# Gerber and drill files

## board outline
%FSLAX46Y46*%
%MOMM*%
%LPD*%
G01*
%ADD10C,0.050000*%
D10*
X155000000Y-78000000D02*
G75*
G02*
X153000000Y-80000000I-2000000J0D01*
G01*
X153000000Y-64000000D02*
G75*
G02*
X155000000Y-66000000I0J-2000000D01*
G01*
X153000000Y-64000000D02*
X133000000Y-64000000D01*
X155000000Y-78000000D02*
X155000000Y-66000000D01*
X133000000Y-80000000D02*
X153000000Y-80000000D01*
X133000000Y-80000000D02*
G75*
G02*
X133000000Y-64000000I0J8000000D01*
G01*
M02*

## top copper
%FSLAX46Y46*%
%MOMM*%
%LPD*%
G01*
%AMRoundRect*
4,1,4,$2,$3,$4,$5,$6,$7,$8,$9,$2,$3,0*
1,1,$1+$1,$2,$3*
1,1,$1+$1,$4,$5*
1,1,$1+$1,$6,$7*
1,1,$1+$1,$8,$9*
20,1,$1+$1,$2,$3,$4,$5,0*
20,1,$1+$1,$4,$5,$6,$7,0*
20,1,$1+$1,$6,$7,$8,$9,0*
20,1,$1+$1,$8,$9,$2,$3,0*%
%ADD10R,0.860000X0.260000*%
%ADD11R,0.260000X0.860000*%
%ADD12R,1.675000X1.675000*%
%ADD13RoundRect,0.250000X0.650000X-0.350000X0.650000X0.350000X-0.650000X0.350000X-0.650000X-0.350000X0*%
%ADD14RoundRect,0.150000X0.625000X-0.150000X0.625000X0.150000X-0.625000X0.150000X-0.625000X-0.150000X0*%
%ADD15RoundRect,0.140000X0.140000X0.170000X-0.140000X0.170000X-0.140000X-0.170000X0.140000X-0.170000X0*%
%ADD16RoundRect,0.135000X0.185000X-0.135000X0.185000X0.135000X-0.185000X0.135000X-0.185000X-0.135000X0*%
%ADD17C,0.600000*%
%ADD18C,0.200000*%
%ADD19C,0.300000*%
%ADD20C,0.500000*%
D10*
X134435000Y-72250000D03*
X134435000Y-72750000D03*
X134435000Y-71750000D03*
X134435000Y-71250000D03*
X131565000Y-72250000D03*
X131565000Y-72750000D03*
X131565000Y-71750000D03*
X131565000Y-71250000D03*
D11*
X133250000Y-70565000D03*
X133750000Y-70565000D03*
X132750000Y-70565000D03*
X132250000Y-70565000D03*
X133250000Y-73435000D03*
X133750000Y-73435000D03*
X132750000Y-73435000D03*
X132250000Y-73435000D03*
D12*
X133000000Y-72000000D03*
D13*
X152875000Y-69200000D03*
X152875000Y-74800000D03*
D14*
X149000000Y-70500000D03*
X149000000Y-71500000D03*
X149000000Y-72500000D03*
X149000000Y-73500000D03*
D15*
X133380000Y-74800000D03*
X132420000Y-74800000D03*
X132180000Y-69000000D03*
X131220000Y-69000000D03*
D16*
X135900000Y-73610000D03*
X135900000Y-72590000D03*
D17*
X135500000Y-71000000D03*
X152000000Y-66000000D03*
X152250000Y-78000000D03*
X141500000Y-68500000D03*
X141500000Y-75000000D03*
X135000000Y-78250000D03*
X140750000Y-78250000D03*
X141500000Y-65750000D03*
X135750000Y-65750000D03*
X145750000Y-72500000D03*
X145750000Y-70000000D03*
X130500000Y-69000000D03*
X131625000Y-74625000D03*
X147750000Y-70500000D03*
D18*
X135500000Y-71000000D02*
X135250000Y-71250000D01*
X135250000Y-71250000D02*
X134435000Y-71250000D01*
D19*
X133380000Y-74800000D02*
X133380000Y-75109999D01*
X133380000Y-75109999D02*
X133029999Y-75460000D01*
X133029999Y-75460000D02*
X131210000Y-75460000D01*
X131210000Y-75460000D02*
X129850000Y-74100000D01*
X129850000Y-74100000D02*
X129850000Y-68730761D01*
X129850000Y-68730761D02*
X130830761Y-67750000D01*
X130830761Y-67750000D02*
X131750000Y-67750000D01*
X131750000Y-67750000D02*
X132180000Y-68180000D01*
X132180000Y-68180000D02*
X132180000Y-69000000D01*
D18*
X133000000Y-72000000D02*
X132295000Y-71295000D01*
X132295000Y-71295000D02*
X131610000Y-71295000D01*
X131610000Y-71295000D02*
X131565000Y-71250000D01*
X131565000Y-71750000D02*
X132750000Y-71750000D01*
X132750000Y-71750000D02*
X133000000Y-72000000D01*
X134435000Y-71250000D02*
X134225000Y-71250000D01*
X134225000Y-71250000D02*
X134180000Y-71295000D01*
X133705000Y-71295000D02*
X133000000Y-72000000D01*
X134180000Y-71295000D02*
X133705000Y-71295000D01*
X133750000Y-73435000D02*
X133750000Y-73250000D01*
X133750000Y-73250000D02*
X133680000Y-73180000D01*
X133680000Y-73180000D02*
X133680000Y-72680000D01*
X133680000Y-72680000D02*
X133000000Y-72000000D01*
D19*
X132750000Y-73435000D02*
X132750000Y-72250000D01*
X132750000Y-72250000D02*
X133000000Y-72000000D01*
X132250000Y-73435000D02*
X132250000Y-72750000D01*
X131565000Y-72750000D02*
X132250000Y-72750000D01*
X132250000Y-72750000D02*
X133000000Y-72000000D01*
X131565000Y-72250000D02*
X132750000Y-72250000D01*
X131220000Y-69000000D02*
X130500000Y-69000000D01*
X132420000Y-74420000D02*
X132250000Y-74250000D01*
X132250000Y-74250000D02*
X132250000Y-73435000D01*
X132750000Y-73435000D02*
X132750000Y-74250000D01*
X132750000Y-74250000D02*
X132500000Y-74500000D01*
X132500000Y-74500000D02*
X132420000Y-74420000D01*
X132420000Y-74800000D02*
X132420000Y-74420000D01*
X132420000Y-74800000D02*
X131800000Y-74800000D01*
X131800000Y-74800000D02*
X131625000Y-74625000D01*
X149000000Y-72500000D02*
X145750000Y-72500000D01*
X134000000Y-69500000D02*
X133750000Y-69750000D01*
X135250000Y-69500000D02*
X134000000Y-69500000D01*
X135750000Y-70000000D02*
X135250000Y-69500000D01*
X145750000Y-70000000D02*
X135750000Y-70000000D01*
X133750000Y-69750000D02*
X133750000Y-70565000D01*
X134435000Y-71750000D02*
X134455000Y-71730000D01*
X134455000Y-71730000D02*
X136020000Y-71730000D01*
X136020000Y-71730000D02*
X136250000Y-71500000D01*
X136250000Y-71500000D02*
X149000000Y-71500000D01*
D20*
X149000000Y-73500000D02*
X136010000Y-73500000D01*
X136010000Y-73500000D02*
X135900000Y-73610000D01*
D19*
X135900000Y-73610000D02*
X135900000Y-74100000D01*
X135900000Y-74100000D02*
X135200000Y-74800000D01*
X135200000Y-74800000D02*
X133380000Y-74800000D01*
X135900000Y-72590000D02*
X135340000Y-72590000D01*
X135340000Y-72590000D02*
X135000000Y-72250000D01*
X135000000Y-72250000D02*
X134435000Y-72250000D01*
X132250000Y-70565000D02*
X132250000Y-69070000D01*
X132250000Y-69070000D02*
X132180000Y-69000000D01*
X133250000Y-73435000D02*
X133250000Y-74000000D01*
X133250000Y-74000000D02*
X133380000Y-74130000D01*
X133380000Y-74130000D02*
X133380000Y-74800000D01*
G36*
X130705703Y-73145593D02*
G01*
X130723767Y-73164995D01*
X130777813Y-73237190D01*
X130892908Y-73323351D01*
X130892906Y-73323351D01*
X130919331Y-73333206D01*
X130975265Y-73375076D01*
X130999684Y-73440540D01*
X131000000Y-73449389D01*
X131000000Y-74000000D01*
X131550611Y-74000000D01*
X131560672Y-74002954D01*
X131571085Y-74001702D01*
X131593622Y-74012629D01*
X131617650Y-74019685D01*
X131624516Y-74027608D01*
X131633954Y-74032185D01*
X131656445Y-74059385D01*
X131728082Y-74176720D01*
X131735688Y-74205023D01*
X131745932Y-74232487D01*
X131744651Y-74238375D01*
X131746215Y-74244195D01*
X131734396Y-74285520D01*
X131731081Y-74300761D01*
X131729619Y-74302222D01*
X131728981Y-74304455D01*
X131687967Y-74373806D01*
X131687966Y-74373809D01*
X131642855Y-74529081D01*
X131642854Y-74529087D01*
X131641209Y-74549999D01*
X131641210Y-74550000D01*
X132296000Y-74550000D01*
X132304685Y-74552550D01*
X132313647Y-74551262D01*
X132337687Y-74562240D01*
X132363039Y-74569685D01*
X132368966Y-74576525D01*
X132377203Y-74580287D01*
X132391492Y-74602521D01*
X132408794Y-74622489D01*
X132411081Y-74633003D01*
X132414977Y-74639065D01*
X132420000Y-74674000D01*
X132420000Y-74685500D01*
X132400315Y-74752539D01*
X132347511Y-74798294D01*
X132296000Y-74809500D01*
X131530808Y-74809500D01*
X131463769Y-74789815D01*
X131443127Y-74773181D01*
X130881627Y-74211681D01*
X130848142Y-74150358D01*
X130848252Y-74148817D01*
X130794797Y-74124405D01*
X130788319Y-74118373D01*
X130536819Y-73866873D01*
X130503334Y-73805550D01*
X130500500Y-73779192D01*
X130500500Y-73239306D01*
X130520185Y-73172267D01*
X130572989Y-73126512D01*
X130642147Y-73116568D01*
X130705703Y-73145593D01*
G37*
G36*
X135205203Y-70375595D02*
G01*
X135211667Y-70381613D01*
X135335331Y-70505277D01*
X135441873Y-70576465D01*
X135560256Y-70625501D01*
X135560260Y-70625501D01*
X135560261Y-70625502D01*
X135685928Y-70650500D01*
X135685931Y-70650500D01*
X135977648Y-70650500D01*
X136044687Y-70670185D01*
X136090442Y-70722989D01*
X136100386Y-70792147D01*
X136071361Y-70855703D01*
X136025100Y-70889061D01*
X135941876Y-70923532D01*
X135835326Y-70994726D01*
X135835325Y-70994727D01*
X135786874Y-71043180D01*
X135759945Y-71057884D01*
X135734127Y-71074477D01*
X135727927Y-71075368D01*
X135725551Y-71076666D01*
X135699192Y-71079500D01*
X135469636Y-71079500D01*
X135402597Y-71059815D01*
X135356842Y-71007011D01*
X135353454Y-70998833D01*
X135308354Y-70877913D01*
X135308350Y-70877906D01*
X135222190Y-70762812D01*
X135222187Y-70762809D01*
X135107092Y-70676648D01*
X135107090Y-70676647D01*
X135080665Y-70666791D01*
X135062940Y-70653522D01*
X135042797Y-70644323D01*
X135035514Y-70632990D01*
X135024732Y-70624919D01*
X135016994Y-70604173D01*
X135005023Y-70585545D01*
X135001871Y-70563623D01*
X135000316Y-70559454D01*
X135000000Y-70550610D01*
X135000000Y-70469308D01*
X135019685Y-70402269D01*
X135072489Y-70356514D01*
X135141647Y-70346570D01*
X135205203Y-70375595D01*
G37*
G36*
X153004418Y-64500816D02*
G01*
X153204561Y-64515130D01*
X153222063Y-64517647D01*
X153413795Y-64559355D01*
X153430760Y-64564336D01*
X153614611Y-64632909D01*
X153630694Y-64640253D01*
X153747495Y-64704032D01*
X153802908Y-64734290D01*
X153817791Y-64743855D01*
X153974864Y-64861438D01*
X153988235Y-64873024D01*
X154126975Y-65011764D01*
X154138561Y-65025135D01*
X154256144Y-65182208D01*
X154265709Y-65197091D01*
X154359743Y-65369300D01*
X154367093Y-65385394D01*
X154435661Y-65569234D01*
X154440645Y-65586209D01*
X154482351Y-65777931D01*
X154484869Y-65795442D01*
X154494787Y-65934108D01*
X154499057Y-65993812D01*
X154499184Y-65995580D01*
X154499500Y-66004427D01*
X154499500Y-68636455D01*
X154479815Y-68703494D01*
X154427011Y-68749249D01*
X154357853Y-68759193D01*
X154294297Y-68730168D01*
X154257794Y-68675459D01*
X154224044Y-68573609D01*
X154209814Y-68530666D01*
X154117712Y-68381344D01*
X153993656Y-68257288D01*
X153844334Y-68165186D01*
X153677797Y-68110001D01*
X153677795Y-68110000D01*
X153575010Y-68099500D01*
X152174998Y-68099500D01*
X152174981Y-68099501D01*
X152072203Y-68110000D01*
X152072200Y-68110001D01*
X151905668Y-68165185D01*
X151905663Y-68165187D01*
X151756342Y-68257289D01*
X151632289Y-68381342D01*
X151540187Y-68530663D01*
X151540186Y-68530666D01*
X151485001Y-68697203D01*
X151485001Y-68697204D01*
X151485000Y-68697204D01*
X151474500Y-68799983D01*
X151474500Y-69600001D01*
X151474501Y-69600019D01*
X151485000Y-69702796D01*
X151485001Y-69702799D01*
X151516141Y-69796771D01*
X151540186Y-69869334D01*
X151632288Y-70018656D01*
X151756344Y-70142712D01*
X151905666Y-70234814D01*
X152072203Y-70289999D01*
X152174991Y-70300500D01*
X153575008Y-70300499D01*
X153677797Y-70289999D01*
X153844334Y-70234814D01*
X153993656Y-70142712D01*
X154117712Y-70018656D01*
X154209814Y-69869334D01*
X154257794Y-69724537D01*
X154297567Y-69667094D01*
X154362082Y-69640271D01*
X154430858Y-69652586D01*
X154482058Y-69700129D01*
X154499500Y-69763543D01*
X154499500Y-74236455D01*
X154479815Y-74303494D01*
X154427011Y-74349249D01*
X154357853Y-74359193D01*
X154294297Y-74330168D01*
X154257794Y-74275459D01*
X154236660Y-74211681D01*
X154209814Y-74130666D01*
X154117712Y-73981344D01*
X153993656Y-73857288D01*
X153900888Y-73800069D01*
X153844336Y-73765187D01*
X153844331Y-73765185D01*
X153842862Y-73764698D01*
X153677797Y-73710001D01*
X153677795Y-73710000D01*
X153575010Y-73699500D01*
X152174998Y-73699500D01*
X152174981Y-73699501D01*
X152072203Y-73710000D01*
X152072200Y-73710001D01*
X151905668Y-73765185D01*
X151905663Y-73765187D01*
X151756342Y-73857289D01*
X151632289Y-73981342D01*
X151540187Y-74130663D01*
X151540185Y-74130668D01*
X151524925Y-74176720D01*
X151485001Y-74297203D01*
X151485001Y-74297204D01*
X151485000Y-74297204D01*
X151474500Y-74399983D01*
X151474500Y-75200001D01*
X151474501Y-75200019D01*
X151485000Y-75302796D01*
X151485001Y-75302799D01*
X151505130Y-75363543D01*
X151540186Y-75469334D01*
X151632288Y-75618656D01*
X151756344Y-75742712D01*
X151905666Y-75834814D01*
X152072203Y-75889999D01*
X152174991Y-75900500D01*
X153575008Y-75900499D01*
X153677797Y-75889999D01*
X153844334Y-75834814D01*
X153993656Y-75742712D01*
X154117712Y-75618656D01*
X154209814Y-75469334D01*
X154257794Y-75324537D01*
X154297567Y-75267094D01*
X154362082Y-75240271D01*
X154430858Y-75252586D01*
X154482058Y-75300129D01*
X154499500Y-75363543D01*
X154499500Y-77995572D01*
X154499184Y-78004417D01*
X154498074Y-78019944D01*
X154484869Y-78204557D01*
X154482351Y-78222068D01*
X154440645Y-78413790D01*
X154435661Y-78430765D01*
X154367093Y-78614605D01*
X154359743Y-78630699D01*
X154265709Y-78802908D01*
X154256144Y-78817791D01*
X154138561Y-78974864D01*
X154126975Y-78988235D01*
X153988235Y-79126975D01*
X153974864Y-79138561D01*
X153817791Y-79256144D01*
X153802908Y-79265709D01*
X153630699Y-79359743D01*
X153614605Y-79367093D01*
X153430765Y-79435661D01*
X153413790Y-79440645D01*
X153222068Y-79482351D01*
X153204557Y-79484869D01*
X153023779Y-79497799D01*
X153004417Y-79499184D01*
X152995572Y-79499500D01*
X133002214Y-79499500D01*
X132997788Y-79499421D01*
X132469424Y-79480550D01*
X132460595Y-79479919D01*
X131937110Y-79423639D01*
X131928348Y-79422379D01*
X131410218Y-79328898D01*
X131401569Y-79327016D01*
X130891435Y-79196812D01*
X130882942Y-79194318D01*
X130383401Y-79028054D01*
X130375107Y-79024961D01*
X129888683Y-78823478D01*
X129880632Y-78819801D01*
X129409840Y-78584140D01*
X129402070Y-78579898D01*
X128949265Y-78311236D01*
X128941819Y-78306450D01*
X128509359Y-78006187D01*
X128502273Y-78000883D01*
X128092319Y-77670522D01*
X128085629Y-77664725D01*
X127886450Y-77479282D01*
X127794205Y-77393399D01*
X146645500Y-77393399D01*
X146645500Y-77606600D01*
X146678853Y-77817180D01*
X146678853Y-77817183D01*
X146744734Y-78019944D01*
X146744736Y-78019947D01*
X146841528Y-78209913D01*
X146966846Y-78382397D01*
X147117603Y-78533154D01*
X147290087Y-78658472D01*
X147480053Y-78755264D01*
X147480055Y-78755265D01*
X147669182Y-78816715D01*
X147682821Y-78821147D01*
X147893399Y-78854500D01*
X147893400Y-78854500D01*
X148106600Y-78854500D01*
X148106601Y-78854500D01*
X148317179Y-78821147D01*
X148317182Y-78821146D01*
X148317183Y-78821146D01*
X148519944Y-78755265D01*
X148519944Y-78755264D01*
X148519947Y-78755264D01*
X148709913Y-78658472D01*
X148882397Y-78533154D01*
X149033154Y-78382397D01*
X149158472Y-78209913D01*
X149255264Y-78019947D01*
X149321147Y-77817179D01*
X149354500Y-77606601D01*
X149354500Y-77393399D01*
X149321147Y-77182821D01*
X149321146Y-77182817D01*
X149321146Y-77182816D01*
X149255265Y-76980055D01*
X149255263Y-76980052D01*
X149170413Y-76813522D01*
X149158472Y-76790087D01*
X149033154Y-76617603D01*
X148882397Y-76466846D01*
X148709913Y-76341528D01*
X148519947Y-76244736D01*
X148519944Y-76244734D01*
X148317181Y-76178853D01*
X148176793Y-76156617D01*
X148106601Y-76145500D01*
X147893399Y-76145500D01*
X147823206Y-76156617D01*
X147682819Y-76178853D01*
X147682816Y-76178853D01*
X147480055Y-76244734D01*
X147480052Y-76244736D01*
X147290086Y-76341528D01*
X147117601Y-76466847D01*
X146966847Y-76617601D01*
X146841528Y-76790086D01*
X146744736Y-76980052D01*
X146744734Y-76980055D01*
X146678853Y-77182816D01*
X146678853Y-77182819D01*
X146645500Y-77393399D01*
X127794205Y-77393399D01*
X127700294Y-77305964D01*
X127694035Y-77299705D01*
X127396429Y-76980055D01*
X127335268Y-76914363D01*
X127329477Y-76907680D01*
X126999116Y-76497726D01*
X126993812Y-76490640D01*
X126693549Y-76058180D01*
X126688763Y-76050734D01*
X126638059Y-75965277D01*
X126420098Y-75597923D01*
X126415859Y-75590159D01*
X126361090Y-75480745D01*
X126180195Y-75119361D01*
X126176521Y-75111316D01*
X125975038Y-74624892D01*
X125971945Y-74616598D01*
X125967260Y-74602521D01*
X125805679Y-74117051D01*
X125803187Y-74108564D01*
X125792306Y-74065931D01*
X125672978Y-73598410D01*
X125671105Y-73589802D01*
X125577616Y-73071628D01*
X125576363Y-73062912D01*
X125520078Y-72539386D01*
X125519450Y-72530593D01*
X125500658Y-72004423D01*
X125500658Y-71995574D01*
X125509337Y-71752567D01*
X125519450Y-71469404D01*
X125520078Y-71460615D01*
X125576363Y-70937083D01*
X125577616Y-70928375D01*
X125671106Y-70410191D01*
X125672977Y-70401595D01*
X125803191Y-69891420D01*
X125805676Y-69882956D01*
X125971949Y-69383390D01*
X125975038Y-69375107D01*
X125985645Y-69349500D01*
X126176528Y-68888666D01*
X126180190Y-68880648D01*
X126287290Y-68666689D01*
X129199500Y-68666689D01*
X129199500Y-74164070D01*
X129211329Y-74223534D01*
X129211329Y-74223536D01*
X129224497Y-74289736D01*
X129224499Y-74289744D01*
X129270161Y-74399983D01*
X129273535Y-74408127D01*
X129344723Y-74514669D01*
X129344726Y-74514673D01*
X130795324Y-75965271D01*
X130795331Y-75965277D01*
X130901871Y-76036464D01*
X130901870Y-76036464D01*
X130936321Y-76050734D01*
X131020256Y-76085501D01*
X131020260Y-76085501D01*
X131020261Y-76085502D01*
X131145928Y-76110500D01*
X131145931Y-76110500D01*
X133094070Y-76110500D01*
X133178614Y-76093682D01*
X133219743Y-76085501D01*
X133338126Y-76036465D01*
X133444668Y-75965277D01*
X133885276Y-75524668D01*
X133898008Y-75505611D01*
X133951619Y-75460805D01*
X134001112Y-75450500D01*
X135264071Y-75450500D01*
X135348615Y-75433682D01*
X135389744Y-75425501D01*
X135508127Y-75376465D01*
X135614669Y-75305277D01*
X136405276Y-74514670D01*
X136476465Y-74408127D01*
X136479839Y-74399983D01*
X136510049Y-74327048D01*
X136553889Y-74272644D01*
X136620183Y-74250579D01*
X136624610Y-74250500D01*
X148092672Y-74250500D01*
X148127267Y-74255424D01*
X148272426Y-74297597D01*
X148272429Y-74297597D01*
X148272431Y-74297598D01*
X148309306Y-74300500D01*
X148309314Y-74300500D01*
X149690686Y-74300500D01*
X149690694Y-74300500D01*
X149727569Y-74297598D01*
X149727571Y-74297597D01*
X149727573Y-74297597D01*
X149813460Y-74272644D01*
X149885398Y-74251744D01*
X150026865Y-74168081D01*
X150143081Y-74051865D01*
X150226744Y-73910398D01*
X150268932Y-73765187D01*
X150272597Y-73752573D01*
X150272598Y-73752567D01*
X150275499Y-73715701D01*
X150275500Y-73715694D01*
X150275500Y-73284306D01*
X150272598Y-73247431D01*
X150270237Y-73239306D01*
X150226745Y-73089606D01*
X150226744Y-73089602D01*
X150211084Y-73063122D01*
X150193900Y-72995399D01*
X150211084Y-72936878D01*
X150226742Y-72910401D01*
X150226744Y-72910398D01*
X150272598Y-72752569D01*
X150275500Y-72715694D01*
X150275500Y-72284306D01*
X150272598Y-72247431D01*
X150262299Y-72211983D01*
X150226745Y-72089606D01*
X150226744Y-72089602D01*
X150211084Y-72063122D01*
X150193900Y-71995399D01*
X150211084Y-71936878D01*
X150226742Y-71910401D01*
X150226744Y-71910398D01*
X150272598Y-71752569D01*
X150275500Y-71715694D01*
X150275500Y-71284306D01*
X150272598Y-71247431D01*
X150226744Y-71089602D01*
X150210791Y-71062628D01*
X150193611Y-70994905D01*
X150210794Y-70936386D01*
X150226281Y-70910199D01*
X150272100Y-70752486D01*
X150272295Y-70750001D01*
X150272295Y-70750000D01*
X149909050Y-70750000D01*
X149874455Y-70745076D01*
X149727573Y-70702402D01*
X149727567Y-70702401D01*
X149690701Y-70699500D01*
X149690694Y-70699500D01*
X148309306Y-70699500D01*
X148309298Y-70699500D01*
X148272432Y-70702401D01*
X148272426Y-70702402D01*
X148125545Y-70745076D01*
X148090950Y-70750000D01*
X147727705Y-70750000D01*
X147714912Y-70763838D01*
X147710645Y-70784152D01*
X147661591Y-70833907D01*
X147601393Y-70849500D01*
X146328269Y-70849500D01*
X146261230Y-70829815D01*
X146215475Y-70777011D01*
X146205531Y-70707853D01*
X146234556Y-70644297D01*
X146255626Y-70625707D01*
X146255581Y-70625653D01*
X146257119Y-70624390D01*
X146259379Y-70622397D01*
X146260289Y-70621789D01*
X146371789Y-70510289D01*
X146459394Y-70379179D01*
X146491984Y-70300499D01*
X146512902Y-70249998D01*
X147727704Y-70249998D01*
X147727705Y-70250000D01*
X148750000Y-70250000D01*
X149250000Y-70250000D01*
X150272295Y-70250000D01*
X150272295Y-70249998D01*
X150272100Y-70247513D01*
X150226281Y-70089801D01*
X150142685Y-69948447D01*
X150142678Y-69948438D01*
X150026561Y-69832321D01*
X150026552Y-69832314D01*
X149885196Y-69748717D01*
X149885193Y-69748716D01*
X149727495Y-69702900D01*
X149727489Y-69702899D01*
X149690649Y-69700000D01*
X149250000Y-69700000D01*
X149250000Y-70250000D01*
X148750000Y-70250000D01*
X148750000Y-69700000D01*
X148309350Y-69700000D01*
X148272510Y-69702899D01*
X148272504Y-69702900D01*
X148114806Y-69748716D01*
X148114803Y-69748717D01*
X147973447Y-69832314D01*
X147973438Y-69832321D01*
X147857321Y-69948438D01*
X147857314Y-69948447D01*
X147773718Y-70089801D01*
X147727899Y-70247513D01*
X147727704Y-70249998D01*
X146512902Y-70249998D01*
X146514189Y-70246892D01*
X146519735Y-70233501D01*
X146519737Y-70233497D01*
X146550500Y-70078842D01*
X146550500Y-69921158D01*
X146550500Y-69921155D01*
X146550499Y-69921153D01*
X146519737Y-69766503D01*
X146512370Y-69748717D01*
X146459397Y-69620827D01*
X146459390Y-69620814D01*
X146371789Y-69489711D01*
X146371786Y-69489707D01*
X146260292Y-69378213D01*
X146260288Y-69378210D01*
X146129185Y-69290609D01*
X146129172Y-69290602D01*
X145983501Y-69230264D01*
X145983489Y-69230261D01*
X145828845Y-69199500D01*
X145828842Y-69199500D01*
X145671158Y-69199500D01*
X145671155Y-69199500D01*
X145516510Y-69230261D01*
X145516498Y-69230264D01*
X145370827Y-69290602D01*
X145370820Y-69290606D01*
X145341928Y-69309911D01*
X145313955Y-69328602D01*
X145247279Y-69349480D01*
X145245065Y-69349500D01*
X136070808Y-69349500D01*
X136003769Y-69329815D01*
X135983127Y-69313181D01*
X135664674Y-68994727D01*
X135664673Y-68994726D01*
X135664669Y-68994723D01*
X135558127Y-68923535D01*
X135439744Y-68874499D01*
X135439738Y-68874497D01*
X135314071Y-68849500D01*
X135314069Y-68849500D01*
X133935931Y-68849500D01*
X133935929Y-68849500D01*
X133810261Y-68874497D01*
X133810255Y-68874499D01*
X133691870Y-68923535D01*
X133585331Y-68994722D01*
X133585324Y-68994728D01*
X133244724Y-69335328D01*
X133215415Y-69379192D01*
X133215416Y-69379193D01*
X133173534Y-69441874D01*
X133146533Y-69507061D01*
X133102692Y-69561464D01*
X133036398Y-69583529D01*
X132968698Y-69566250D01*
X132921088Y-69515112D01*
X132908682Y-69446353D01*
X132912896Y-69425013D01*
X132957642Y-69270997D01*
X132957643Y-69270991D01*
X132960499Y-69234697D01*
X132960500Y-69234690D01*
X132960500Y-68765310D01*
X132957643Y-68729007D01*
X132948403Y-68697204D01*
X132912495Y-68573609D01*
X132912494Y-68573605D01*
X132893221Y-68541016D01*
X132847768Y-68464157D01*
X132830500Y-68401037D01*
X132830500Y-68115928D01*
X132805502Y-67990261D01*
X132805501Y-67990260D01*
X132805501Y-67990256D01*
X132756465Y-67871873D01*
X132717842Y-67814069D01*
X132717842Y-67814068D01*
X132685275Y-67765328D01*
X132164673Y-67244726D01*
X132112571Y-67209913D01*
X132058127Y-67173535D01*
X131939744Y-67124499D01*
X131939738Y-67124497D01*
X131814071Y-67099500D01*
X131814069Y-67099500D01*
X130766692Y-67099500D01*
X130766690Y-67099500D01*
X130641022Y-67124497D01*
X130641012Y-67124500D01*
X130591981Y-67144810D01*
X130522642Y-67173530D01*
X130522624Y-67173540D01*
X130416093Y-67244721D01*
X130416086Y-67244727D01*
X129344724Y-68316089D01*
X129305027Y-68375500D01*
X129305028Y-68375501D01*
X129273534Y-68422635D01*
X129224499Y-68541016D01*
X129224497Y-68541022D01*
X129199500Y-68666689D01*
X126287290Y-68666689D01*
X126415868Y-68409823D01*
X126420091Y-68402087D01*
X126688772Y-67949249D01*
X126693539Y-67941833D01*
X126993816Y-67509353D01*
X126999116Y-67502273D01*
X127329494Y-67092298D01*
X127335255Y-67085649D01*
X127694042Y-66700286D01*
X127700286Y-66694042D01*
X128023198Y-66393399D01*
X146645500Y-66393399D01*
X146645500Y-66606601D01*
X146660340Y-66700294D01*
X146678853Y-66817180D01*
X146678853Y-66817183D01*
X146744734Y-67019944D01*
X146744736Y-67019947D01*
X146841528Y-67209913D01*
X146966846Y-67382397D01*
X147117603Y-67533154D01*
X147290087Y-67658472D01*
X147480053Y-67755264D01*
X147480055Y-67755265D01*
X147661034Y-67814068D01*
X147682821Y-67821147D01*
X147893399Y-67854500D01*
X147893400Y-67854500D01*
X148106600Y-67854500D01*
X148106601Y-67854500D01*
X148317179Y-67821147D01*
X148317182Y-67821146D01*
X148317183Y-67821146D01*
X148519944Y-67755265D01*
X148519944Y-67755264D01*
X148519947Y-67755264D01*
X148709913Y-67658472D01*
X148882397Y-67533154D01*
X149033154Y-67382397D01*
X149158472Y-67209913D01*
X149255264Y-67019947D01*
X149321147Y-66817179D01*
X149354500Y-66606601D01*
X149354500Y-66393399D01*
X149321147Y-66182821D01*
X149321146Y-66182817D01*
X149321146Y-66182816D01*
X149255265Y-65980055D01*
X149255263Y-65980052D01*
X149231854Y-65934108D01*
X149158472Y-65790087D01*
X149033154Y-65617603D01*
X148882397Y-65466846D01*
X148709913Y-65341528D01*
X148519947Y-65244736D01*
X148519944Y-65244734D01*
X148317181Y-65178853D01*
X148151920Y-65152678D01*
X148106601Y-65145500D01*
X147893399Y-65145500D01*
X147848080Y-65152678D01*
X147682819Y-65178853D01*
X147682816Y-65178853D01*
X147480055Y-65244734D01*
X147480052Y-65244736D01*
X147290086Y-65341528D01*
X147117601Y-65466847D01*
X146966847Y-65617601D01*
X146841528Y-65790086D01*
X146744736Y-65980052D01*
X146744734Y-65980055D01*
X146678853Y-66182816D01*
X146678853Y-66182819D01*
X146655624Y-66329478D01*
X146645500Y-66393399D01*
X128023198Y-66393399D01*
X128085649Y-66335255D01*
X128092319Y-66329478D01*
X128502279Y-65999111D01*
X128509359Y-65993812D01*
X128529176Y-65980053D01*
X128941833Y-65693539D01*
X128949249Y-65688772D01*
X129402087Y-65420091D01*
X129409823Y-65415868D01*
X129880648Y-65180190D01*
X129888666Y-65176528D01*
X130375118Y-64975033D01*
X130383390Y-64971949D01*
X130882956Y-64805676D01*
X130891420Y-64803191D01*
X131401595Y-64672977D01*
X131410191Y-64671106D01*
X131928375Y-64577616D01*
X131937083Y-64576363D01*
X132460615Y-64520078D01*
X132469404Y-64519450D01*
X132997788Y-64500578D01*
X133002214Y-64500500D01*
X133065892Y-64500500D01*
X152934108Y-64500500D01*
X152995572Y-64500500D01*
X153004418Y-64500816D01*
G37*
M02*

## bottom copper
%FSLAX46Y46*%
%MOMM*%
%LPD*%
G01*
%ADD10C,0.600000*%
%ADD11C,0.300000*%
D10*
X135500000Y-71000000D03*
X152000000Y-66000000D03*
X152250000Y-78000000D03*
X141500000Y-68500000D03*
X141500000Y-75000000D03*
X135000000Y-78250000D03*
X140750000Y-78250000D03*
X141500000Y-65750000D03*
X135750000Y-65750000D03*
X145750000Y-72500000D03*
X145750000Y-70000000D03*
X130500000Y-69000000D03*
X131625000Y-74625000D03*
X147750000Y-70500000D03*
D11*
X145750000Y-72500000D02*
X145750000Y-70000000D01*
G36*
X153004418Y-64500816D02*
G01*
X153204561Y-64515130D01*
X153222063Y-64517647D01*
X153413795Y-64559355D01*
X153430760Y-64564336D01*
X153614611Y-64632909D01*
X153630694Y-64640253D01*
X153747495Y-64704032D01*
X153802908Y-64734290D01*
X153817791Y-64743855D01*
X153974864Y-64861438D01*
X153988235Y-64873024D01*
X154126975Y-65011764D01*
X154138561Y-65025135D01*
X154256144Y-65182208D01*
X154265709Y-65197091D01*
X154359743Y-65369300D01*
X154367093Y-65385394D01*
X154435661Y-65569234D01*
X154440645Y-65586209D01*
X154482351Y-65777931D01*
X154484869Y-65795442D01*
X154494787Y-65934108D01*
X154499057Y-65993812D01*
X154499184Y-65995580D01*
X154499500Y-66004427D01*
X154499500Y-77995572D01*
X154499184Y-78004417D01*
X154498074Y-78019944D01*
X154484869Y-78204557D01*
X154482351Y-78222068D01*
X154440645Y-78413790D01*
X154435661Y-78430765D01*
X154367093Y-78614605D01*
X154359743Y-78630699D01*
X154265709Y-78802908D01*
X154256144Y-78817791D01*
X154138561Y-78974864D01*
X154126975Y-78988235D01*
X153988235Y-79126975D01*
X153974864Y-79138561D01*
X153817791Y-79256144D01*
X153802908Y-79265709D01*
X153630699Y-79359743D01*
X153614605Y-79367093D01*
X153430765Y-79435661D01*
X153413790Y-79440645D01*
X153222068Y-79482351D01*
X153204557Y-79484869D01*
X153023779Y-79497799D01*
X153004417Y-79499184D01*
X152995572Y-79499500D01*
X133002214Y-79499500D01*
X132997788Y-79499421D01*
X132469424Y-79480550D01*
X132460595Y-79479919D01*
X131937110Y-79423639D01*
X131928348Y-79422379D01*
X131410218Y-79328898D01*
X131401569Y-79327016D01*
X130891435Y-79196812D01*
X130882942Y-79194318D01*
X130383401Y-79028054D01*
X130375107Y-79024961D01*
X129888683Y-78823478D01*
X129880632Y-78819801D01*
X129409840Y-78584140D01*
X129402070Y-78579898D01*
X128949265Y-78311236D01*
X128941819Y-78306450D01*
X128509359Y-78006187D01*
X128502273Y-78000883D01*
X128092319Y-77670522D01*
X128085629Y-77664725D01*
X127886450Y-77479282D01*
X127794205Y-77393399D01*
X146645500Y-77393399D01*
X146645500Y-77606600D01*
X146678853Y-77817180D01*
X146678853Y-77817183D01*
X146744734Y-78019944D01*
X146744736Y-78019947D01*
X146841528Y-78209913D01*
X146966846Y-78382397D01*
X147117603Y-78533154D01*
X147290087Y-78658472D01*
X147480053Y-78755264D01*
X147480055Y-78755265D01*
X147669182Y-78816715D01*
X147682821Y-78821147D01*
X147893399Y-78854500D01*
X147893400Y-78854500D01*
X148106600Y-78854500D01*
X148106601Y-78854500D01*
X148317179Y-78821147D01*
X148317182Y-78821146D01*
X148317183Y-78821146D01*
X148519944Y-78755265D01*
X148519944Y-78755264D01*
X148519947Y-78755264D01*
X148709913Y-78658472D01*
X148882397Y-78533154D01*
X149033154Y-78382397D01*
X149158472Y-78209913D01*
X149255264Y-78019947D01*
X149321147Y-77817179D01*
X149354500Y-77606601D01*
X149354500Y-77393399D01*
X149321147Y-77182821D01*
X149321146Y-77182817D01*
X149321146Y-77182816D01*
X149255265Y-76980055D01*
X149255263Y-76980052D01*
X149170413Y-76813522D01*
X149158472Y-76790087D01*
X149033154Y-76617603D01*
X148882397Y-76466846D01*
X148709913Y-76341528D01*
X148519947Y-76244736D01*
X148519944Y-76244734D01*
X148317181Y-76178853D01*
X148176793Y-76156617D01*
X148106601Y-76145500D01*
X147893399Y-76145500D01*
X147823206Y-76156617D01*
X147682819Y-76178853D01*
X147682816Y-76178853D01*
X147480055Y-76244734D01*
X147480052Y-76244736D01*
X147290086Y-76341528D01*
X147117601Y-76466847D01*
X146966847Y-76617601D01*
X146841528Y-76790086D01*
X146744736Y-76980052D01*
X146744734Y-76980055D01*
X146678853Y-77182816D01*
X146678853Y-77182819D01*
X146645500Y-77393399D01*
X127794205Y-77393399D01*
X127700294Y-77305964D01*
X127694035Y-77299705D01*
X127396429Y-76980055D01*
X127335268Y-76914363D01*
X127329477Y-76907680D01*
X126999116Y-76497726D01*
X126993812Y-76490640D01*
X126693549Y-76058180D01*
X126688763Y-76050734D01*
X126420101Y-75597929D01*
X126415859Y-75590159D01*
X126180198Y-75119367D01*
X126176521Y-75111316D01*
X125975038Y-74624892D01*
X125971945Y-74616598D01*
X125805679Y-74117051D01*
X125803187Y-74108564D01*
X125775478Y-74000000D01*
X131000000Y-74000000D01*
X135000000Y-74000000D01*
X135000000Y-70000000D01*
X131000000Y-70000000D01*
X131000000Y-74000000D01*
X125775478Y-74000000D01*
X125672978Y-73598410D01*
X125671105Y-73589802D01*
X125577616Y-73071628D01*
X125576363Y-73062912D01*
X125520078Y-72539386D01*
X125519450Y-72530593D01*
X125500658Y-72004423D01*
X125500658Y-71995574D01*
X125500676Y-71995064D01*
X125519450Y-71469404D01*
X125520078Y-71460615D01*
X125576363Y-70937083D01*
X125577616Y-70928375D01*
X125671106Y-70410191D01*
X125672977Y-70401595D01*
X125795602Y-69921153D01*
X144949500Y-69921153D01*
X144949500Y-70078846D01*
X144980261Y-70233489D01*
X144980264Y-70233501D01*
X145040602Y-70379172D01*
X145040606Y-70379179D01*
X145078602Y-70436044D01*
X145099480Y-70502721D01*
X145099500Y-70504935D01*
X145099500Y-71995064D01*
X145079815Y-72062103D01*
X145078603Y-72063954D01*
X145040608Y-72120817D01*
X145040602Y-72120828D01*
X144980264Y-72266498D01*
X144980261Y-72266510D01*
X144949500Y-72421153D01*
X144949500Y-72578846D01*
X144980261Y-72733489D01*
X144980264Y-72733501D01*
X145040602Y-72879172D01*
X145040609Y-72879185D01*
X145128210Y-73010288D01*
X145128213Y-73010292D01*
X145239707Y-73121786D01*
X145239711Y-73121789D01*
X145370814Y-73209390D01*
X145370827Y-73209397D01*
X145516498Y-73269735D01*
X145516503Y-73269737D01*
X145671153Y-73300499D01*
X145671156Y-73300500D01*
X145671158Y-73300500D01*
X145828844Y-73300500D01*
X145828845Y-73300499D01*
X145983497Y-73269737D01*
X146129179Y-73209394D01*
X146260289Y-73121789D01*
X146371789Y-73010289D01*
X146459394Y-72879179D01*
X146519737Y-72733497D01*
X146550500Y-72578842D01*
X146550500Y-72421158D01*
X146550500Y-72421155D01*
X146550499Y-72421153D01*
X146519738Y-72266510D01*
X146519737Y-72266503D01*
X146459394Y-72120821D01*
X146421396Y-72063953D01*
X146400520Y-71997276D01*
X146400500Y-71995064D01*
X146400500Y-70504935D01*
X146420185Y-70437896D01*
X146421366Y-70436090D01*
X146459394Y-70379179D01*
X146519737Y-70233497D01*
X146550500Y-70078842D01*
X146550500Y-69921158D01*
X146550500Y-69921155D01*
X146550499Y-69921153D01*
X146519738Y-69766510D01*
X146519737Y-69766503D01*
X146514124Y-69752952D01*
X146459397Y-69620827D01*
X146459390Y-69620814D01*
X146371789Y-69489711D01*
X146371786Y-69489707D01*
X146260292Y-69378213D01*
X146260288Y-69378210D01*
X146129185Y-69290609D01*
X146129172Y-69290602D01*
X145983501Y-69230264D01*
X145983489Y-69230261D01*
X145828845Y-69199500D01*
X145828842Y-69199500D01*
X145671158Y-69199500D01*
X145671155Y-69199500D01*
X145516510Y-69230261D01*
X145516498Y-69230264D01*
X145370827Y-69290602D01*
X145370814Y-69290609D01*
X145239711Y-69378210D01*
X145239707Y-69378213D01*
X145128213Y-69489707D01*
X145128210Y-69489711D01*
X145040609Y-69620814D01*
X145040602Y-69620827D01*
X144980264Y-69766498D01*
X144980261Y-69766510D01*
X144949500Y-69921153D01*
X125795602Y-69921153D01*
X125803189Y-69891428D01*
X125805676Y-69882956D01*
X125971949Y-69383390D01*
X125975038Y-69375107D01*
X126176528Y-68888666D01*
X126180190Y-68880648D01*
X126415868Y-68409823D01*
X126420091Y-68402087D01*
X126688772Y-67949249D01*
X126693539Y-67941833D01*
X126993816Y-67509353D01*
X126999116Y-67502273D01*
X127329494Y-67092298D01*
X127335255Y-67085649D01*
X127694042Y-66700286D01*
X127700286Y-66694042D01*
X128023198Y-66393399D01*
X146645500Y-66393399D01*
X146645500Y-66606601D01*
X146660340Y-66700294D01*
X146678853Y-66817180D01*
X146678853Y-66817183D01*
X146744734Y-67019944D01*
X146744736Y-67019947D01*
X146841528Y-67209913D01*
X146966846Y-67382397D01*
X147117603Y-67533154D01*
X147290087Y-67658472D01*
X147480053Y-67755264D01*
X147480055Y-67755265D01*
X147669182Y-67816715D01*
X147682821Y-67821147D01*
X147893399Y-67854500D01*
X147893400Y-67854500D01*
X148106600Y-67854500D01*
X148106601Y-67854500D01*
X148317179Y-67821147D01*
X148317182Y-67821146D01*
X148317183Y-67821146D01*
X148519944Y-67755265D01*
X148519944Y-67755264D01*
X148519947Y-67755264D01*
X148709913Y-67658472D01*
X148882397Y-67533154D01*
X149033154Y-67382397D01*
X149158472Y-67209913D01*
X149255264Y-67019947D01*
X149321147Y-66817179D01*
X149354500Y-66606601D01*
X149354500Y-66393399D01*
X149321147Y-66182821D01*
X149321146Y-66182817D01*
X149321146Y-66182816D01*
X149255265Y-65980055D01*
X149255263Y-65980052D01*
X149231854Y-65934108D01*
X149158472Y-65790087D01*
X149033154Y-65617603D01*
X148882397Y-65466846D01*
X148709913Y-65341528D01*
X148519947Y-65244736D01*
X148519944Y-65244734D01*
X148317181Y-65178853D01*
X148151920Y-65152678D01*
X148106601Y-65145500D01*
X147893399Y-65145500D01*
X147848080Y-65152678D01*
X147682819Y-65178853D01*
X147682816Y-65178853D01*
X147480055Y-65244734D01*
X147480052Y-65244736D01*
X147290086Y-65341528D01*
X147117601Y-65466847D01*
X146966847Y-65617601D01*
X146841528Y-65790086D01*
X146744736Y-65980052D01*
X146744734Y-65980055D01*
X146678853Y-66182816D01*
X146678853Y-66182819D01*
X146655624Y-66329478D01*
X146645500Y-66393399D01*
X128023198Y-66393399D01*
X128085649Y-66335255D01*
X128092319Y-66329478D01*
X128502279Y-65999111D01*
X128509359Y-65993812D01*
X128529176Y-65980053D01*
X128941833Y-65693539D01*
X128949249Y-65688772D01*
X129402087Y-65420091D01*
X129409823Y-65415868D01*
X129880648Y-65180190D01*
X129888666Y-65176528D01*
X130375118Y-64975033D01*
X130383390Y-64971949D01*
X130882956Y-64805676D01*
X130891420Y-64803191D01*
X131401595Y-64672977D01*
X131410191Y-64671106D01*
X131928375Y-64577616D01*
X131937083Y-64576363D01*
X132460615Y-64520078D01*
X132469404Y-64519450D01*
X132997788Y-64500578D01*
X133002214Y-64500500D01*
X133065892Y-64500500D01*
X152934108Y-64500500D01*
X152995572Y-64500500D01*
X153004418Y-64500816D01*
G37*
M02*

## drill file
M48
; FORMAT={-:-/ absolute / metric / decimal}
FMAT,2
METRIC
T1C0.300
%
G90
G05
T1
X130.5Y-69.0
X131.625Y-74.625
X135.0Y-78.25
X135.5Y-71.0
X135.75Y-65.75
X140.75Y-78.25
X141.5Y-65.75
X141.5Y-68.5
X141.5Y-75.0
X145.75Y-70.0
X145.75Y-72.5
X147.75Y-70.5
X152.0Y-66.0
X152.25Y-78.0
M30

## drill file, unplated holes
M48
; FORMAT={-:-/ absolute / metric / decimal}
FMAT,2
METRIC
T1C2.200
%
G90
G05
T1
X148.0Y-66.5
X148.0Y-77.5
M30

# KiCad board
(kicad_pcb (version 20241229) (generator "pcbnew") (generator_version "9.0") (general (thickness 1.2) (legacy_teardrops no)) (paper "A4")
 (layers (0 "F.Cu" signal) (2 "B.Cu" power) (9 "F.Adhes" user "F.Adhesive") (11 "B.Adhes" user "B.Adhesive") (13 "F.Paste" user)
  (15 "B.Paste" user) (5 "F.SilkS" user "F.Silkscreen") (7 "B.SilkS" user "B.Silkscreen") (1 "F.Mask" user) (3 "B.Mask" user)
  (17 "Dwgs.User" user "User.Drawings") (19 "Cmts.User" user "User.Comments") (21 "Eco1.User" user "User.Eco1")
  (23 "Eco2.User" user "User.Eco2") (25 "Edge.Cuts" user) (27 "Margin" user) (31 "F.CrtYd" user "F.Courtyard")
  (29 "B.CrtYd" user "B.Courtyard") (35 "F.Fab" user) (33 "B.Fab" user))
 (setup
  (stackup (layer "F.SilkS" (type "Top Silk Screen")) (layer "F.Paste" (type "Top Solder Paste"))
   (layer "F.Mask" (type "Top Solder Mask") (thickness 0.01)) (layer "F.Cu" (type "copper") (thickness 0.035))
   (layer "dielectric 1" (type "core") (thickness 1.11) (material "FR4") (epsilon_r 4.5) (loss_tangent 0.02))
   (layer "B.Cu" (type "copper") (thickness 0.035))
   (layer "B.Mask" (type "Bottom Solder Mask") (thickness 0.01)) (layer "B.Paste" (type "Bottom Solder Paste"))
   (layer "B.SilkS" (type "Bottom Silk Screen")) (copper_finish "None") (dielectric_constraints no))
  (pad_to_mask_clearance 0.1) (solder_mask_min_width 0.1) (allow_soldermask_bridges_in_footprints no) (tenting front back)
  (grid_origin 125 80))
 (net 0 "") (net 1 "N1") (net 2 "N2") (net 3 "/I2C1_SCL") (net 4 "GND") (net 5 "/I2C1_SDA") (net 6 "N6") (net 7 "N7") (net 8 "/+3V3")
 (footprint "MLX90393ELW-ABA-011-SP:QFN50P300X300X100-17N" (layer "F.Cu") (at 133 72 180)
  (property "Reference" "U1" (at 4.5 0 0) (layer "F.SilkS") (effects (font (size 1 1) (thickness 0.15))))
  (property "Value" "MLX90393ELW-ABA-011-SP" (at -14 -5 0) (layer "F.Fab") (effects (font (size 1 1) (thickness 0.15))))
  (pad "1" smd rect (at -1.435 -0.75 180) (size 0.86 0.26) (layers "F.Cu" "F.Mask" "F.Paste") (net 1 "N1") (solder_mask_margin 0.102))
  (pad "2" smd rect (at -1.435 -0.25 180) (size 0.86 0.26) (layers "F.Cu" "F.Mask" "F.Paste") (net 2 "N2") (solder_mask_margin 0.102))
  (pad "3" smd rect (at -1.435 0.25 180) (size 0.86 0.26) (layers "F.Cu" "F.Mask" "F.Paste") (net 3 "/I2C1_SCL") (solder_mask_margin 0.102))
  (pad "4" smd rect (at -1.435 0.75 180) (size 0.86 0.26) (layers "F.Cu" "F.Mask" "F.Paste") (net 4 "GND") (solder_mask_margin 0.102))
  (pad "5" smd rect (at -0.75 1.435 180) (size 0.26 0.86) (layers "F.Cu" "F.Mask" "F.Paste") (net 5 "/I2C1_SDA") (solder_mask_margin 0.102))
  (pad "6" smd rect (at -0.25 1.435 180) (size 0.26 0.86) (layers "F.Cu" "F.Mask" "F.Paste") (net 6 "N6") (solder_mask_margin 0.102))
  (pad "7" smd rect (at 0.25 1.435 180) (size 0.26 0.86) (layers "F.Cu" "F.Mask" "F.Paste") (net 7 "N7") (solder_mask_margin 0.102))
  (pad "8" smd rect (at 0.75 1.435 180) (size 0.26 0.86) (layers "F.Cu" "F.Mask" "F.Paste") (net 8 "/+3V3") (solder_mask_margin 0.102))
  (pad "9" smd rect (at 1.435 0.75 180) (size 0.86 0.26) (layers "F.Cu" "F.Mask" "F.Paste") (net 4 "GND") (solder_mask_margin 0.102))
  (pad "10" smd rect (at 1.435 0.25 180) (size 0.86 0.26) (layers "F.Cu" "F.Mask" "F.Paste") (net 4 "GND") (solder_mask_margin 0.102))
  (pad "11" smd rect (at 1.435 -0.25 180) (size 0.86 0.26) (layers "F.Cu" "F.Mask" "F.Paste") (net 4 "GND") (solder_mask_margin 0.102))
  (pad "12" smd rect (at 1.435 -0.75 180) (size 0.86 0.26) (layers "F.Cu" "F.Mask" "F.Paste") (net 4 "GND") (solder_mask_margin 0.102))
  (pad "13" smd rect (at 0.75 -1.435 180) (size 0.26 0.86) (layers "F.Cu" "F.Mask" "F.Paste") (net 4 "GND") (solder_mask_margin 0.102))
  (pad "14" smd rect (at 0.25 -1.435 180) (size 0.26 0.86) (layers "F.Cu" "F.Mask" "F.Paste") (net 4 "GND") (solder_mask_margin 0.102))
  (pad "15" smd rect (at -0.25 -1.435 180) (size 0.26 0.86) (layers "F.Cu" "F.Mask" "F.Paste") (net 8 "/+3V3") (solder_mask_margin 0.102))
  (pad "16" smd rect (at -0.75 -1.435 180) (size 0.26 0.86) (layers "F.Cu" "F.Mask" "F.Paste") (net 4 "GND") (solder_mask_margin 0.102))
  (pad "17" smd rect (at 0 0 180) (size 1.675 1.675) (layers "F.Cu" "F.Mask") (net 4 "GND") (solder_mask_margin 0.102) (clearance 0.1675)))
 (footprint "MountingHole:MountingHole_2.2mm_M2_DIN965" (layer "F.Cu") (at 148 66.5)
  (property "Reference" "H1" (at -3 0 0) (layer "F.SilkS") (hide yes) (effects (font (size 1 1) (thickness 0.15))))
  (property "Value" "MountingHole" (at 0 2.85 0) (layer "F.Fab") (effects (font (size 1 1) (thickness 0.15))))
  (pad "" np_thru_hole circle (at 0 0) (size 2.2 2.2) (drill 2.2) (layers "*.Cu" "*.Mask")))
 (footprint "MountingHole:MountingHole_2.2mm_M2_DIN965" (layer "F.Cu") (at 148 77.5)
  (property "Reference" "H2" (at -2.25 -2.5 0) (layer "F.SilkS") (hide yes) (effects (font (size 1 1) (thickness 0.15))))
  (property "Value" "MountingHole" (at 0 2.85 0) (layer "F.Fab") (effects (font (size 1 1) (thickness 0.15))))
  (pad "" np_thru_hole circle (at 0 0) (size 2.2 2.2) (drill 2.2) (layers "*.Cu" "*.Mask")))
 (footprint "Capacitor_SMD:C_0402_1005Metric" (layer "F.Cu") (at 131.7 69 180)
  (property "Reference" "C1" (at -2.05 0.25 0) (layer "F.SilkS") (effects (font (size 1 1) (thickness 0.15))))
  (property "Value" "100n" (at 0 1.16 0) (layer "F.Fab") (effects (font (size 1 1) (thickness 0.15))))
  (pad "1" smd roundrect (at -0.48 0 180) (size 0.56 0.62) (layers "F.Cu" "F.Mask" "F.Paste") (roundrect_rratio 0.25) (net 8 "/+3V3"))
  (pad "2" smd roundrect (at 0.48 0 180) (size 0.56 0.62) (layers "F.Cu" "F.Mask" "F.Paste") (roundrect_rratio 0.25) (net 4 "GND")))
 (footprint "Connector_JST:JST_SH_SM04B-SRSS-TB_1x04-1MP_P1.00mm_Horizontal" (layer "F.Cu") (at 151 72 90)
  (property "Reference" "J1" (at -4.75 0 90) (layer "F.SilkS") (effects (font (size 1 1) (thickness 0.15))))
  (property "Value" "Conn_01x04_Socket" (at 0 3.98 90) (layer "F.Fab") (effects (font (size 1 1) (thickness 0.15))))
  (pad "1" smd roundrect (at -1.5 -2 90) (size 0.6 1.55) (layers "F.Cu" "F.Mask" "F.Paste") (roundrect_rratio 0.25) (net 8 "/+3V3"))
  (pad "2" smd roundrect (at -0.5 -2 90) (size 0.6 1.55) (layers "F.Cu" "F.Mask" "F.Paste") (roundrect_rratio 0.25) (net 5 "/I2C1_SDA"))
  (pad "3" smd roundrect (at 0.5 -2 90) (size 0.6 1.55) (layers "F.Cu" "F.Mask" "F.Paste") (roundrect_rratio 0.25) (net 3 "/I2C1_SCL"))
  (pad "4" smd roundrect (at 1.5 -2 90) (size 0.6 1.55) (layers "F.Cu" "F.Mask" "F.Paste") (roundrect_rratio 0.25) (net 4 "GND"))
  (pad "MP" smd roundrect (at -2.8 1.875 90) (size 1.2 1.8) (layers "F.Cu" "F.Mask" "F.Paste") (roundrect_rratio 0.208333))
  (pad "MP" smd roundrect (at 2.8 1.875 90) (size 1.2 1.8) (layers "F.Cu" "F.Mask" "F.Paste") (roundrect_rratio 0.208333)))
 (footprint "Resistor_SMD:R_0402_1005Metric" (layer "F.Cu") (at 135.9 73.1 90)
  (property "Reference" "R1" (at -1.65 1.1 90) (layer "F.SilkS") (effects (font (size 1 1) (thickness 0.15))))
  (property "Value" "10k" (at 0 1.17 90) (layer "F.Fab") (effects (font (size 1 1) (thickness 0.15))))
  (pad "1" smd roundrect (at -0.51 0 90) (size 0.54 0.64) (layers "F.Cu" "F.Mask" "F.Paste") (roundrect_rratio 0.25) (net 8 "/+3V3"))
  (pad "2" smd roundrect (at 0.51 0 90) (size 0.54 0.64) (layers "F.Cu" "F.Mask" "F.Paste") (roundrect_rratio 0.25) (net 2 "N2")))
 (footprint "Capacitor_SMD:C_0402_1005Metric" (layer "F.Cu") (at 132.9 74.8 180)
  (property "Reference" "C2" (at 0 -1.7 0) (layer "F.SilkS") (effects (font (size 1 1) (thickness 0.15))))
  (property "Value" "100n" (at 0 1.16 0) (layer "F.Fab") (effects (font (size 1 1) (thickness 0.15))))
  (pad "1" smd roundrect (at -0.48 0 180) (size 0.56 0.62) (layers "F.Cu" "F.Mask" "F.Paste") (roundrect_rratio 0.25) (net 8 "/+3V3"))
  (pad "2" smd roundrect (at 0.48 0 180) (size 0.56 0.62) (layers "F.Cu" "F.Mask" "F.Paste") (roundrect_rratio 0.25) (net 4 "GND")))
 (gr_arc (start 133 80) (mid 125 72) (end 133 64) (stroke (width 0.05) (type default)) (layer "Edge.Cuts"))
 (gr_line (start 133 80) (end 153 80) (stroke (width 0.05) (type default)) (layer "Edge.Cuts"))
 (gr_line (start 153 64) (end 133 64) (stroke (width 0.05) (type default)) (layer "Edge.Cuts"))
 (gr_arc (start 153 64) (mid 154.414214 64.585786) (end 155 66) (stroke (width 0.05) (type default)) (layer "Edge.Cuts"))
 (gr_arc (start 155 78) (mid 154.414214 79.414214) (end 153 80) (stroke (width 0.05) (type default)) (layer "Edge.Cuts"))
 (gr_line (start 155 78) (end 155 66) (stroke (width 0.05) (type default)) (layer "Edge.Cuts"))
 (segment (start 133.38 74.8) (end 133.38 75.109999) (width 0.3) (layer "F.Cu") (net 8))
 (segment (start 136.01 73.5) (end 135.9 73.61) (width 0.5) (layer "F.Cu") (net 8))
 (segment (start 133.38 75.109999) (end 133.029999 75.46) (width 0.3) (layer "F.Cu") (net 8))
 (segment (start 131.75 67.75) (end 132.18 68.18) (width 0.3) (layer "F.Cu") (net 8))
 (segment (start 129.85 74.1) (end 129.85 68.730761) (width 0.3) (layer "F.Cu") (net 8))
 (segment (start 133.25 74) (end 133.38 74.13) (width 0.3) (layer "F.Cu") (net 8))
 (segment (start 132.18 68.18) (end 132.18 69) (width 0.3) (layer "F.Cu") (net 8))
 (segment (start 131.21 75.46) (end 129.85 74.1) (width 0.3) (layer "F.Cu") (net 8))
 (segment (start 135.9 73.61) (end 135.9 74.1) (width 0.3) (layer "F.Cu") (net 8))
 (segment (start 149 73.5) (end 136.01 73.5) (width 0.5) (layer "F.Cu") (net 8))
 (segment (start 135.9 74.1) (end 135.2 74.8) (width 0.3) (layer "F.Cu") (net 8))
 (segment (start 132.25 70.565) (end 132.25 69.07) (width 0.3) (layer "F.Cu") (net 8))
 (segment (start 133.38 74.13) (end 133.38 74.8) (width 0.3) (layer "F.Cu") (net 8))
 (segment (start 132.25 69.07) (end 132.18 69) (width 0.3) (layer "F.Cu") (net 8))
 (segment (start 133.25 73.435) (end 133.25 74) (width 0.3) (layer "F.Cu") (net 8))
 (segment (start 133.029999 75.46) (end 131.21 75.46) (width 0.3) (layer "F.Cu") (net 8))
 (segment (start 130.830761 67.75) (end 131.75 67.75) (width 0.3) (layer "F.Cu") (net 8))
 (segment (start 135.2 74.8) (end 133.38 74.8) (width 0.3) (layer "F.Cu") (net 8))
 (segment (start 129.85 68.730761) (end 130.830761 67.75) (width 0.3) (layer "F.Cu") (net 8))
 (segment (start 132.42 74.42) (end 132.25 74.25) (width 0.3) (layer "F.Cu") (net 4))
 (segment (start 133.68 72.68) (end 133 72) (width 0.2) (layer "F.Cu") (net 4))
 (segment (start 131.565 71.75) (end 132.75 71.75) (width 0.2) (layer "F.Cu") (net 4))
 (segment (start 133.75 73.435) (end 133.75 73.25) (width 0.2) (layer "F.Cu") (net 4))
 (segment (start 131.565 72.75) (end 132.25 72.75) (width 0.3) (layer "F.Cu") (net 4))
 (segment (start 131.61 71.295) (end 131.565 71.25) (width 0.2) (layer "F.Cu") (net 4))
 (segment (start 133.705 71.295) (end 133 72) (width 0.2) (layer "F.Cu") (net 4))
 (segment (start 132.75 74.25) (end 132.5 74.5) (width 0.3) (layer "F.Cu") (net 4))
 (segment (start 132.42 74.8) (end 131.8 74.8) (width 0.3) (layer "F.Cu") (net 4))
 (segment (start 134.225 71.25) (end 134.18 71.295) (width 0.2) (layer "F.Cu") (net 4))
 (segment (start 132.295 71.295) (end 131.61 71.295) (width 0.2) (layer "F.Cu") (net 4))
 (segment (start 133.68 73.18) (end 133.68 72.68) (width 0.2) (layer "F.Cu") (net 4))
 (segment (start 132.25 73.435) (end 132.25 72.75) (width 0.3) (layer "F.Cu") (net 4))
 (segment (start 131.22 69) (end 130.5 69) (width 0.3) (layer "F.Cu") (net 4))
 (segment (start 132.25 74.25) (end 132.25 73.435) (width 0.3) (layer "F.Cu") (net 4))
 (segment (start 134.435 71.25) (end 134.225 71.25) (width 0.2) (layer "F.Cu") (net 4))
 (segment (start 134.18 71.295) (end 133.705 71.295) (width 0.2) (layer "F.Cu") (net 4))
 (segment (start 133 72) (end 132.295 71.295) (width 0.2) (layer "F.Cu") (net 4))
 (segment (start 131.8 74.8) (end 131.625 74.625) (width 0.3) (layer "F.Cu") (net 4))
 (segment (start 135.25 71.25) (end 134.435 71.25) (width 0.2) (layer "F.Cu") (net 4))
 (segment (start 132.75 73.435) (end 132.75 74.25) (width 0.3) (layer "F.Cu") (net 4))
 (segment (start 132.75 73.435) (end 132.75 72.25) (width 0.3) (layer "F.Cu") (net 4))
 (segment (start 132.5 74.5) (end 132.42 74.42) (width 0.3) (layer "F.Cu") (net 4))
 (segment (start 133.75 73.25) (end 133.68 73.18) (width 0.2) (layer "F.Cu") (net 4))
 (segment (start 132.25 72.75) (end 133 72) (width 0.3) (layer "F.Cu") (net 4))
 (segment (start 132.75 72.25) (end 133 72) (width 0.3) (layer "F.Cu") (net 4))
 (segment (start 135.5 71) (end 135.25 71.25) (width 0.2) (layer "F.Cu") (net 4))
 (segment (start 132.42 74.8) (end 132.42 74.42) (width 0.3) (layer "F.Cu") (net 4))
 (segment (start 132.75 71.75) (end 133 72) (width 0.2) (layer "F.Cu") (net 4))
 (segment (start 131.565 72.25) (end 132.75 72.25) (width 0.3) (layer "F.Cu") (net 4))
 (via (at 147.75 70.5) (size 0.6) (drill 0.3) (layers "F.Cu" "B.Cu") (free yes) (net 4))
 (via (at 140.75 78.25) (size 0.6) (drill 0.3) (layers "F.Cu" "B.Cu") (free yes) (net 4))
 (via (at 141.5 68.5) (size 0.6) (drill 0.3) (layers "F.Cu" "B.Cu") (free yes) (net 4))
 (via (at 135.5 71) (size 0.6) (drill 0.3) (layers "F.Cu" "B.Cu") (free yes) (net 4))
 (via (at 152.25 78) (size 0.6) (drill 0.3) (layers "F.Cu" "B.Cu") (free yes) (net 4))
 (via (at 152 66) (size 0.6) (drill 0.3) (layers "F.Cu" "B.Cu") (free yes) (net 4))
 (via (at 131.625 74.625) (size 0.6) (drill 0.3) (layers "F.Cu" "B.Cu") (free yes) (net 4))
 (via (at 130.5 69) (size 0.6) (drill 0.3) (layers "F.Cu" "B.Cu") (free yes) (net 4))
 (via (at 135 78.25) (size 0.6) (drill 0.3) (layers "F.Cu" "B.Cu") (free yes) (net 4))
 (via (at 135.75 65.75) (size 0.6) (drill 0.3) (layers "F.Cu" "B.Cu") (free yes) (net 4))
 (via (at 141.5 75) (size 0.6) (drill 0.3) (layers "F.Cu" "B.Cu") (free yes) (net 4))
 (via (at 141.5 65.75) (size 0.6) (drill 0.3) (layers "F.Cu" "B.Cu") (free yes) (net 4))
 (segment (start 134.455 71.73) (end 136.02 71.73) (width 0.3) (layer "F.Cu") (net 3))
 (segment (start 136.25 71.5) (end 149 71.5) (width 0.3) (layer "F.Cu") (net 3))
 (segment (start 136.02 71.73) (end 136.25 71.5) (width 0.3) (layer "F.Cu") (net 3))
 (segment (start 134.435 71.75) (end 134.455 71.73) (width 0.3) (layer "F.Cu") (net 3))
 (segment (start 135.75 70) (end 135.25 69.5) (width 0.3) (layer "F.Cu") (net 5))
 (segment (start 135.25 69.5) (end 134 69.5) (width 0.3) (layer "F.Cu") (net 5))
 (segment (start 133.75 69.75) (end 133.75 70.565) (width 0.3) (layer "F.Cu") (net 5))
 (segment (start 134 69.5) (end 133.75 69.75) (width 0.3) (layer "F.Cu") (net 5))
 (segment (start 145.75 70) (end 135.75 70) (width 0.3) (layer "F.Cu") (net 5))
 (segment (start 149 72.5) (end 145.75 72.5) (width 0.3) (layer "F.Cu") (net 5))
 (via (at 145.75 72.5) (size 0.6) (drill 0.3) (layers "F.Cu" "B.Cu") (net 5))
 (via (at 145.75 70) (size 0.6) (drill 0.3) (layers "F.Cu" "B.Cu") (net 5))
 (segment (start 145.75 72.5) (end 145.75 70) (width 0.3) (layer "B.Cu") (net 5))
 (segment (start 135 72.25) (end 134.435 72.25) (width 0.3) (layer "F.Cu") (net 2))
 (segment (start 135.9 72.59) (end 135.34 72.59) (width 0.3) (layer "F.Cu") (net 2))
 (segment (start 135.34 72.59) (end 135 72.25) (width 0.3) (layer "F.Cu") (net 2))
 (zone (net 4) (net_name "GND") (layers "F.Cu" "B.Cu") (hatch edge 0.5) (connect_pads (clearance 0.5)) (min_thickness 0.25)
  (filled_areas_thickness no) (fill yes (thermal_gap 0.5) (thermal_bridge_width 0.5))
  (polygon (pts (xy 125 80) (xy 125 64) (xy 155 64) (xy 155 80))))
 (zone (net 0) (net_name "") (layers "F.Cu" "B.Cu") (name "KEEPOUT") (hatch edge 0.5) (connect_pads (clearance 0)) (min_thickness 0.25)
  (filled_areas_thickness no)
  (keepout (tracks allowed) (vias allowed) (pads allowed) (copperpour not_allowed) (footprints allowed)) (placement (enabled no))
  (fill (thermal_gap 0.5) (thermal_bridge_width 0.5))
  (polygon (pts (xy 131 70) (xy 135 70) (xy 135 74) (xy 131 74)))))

